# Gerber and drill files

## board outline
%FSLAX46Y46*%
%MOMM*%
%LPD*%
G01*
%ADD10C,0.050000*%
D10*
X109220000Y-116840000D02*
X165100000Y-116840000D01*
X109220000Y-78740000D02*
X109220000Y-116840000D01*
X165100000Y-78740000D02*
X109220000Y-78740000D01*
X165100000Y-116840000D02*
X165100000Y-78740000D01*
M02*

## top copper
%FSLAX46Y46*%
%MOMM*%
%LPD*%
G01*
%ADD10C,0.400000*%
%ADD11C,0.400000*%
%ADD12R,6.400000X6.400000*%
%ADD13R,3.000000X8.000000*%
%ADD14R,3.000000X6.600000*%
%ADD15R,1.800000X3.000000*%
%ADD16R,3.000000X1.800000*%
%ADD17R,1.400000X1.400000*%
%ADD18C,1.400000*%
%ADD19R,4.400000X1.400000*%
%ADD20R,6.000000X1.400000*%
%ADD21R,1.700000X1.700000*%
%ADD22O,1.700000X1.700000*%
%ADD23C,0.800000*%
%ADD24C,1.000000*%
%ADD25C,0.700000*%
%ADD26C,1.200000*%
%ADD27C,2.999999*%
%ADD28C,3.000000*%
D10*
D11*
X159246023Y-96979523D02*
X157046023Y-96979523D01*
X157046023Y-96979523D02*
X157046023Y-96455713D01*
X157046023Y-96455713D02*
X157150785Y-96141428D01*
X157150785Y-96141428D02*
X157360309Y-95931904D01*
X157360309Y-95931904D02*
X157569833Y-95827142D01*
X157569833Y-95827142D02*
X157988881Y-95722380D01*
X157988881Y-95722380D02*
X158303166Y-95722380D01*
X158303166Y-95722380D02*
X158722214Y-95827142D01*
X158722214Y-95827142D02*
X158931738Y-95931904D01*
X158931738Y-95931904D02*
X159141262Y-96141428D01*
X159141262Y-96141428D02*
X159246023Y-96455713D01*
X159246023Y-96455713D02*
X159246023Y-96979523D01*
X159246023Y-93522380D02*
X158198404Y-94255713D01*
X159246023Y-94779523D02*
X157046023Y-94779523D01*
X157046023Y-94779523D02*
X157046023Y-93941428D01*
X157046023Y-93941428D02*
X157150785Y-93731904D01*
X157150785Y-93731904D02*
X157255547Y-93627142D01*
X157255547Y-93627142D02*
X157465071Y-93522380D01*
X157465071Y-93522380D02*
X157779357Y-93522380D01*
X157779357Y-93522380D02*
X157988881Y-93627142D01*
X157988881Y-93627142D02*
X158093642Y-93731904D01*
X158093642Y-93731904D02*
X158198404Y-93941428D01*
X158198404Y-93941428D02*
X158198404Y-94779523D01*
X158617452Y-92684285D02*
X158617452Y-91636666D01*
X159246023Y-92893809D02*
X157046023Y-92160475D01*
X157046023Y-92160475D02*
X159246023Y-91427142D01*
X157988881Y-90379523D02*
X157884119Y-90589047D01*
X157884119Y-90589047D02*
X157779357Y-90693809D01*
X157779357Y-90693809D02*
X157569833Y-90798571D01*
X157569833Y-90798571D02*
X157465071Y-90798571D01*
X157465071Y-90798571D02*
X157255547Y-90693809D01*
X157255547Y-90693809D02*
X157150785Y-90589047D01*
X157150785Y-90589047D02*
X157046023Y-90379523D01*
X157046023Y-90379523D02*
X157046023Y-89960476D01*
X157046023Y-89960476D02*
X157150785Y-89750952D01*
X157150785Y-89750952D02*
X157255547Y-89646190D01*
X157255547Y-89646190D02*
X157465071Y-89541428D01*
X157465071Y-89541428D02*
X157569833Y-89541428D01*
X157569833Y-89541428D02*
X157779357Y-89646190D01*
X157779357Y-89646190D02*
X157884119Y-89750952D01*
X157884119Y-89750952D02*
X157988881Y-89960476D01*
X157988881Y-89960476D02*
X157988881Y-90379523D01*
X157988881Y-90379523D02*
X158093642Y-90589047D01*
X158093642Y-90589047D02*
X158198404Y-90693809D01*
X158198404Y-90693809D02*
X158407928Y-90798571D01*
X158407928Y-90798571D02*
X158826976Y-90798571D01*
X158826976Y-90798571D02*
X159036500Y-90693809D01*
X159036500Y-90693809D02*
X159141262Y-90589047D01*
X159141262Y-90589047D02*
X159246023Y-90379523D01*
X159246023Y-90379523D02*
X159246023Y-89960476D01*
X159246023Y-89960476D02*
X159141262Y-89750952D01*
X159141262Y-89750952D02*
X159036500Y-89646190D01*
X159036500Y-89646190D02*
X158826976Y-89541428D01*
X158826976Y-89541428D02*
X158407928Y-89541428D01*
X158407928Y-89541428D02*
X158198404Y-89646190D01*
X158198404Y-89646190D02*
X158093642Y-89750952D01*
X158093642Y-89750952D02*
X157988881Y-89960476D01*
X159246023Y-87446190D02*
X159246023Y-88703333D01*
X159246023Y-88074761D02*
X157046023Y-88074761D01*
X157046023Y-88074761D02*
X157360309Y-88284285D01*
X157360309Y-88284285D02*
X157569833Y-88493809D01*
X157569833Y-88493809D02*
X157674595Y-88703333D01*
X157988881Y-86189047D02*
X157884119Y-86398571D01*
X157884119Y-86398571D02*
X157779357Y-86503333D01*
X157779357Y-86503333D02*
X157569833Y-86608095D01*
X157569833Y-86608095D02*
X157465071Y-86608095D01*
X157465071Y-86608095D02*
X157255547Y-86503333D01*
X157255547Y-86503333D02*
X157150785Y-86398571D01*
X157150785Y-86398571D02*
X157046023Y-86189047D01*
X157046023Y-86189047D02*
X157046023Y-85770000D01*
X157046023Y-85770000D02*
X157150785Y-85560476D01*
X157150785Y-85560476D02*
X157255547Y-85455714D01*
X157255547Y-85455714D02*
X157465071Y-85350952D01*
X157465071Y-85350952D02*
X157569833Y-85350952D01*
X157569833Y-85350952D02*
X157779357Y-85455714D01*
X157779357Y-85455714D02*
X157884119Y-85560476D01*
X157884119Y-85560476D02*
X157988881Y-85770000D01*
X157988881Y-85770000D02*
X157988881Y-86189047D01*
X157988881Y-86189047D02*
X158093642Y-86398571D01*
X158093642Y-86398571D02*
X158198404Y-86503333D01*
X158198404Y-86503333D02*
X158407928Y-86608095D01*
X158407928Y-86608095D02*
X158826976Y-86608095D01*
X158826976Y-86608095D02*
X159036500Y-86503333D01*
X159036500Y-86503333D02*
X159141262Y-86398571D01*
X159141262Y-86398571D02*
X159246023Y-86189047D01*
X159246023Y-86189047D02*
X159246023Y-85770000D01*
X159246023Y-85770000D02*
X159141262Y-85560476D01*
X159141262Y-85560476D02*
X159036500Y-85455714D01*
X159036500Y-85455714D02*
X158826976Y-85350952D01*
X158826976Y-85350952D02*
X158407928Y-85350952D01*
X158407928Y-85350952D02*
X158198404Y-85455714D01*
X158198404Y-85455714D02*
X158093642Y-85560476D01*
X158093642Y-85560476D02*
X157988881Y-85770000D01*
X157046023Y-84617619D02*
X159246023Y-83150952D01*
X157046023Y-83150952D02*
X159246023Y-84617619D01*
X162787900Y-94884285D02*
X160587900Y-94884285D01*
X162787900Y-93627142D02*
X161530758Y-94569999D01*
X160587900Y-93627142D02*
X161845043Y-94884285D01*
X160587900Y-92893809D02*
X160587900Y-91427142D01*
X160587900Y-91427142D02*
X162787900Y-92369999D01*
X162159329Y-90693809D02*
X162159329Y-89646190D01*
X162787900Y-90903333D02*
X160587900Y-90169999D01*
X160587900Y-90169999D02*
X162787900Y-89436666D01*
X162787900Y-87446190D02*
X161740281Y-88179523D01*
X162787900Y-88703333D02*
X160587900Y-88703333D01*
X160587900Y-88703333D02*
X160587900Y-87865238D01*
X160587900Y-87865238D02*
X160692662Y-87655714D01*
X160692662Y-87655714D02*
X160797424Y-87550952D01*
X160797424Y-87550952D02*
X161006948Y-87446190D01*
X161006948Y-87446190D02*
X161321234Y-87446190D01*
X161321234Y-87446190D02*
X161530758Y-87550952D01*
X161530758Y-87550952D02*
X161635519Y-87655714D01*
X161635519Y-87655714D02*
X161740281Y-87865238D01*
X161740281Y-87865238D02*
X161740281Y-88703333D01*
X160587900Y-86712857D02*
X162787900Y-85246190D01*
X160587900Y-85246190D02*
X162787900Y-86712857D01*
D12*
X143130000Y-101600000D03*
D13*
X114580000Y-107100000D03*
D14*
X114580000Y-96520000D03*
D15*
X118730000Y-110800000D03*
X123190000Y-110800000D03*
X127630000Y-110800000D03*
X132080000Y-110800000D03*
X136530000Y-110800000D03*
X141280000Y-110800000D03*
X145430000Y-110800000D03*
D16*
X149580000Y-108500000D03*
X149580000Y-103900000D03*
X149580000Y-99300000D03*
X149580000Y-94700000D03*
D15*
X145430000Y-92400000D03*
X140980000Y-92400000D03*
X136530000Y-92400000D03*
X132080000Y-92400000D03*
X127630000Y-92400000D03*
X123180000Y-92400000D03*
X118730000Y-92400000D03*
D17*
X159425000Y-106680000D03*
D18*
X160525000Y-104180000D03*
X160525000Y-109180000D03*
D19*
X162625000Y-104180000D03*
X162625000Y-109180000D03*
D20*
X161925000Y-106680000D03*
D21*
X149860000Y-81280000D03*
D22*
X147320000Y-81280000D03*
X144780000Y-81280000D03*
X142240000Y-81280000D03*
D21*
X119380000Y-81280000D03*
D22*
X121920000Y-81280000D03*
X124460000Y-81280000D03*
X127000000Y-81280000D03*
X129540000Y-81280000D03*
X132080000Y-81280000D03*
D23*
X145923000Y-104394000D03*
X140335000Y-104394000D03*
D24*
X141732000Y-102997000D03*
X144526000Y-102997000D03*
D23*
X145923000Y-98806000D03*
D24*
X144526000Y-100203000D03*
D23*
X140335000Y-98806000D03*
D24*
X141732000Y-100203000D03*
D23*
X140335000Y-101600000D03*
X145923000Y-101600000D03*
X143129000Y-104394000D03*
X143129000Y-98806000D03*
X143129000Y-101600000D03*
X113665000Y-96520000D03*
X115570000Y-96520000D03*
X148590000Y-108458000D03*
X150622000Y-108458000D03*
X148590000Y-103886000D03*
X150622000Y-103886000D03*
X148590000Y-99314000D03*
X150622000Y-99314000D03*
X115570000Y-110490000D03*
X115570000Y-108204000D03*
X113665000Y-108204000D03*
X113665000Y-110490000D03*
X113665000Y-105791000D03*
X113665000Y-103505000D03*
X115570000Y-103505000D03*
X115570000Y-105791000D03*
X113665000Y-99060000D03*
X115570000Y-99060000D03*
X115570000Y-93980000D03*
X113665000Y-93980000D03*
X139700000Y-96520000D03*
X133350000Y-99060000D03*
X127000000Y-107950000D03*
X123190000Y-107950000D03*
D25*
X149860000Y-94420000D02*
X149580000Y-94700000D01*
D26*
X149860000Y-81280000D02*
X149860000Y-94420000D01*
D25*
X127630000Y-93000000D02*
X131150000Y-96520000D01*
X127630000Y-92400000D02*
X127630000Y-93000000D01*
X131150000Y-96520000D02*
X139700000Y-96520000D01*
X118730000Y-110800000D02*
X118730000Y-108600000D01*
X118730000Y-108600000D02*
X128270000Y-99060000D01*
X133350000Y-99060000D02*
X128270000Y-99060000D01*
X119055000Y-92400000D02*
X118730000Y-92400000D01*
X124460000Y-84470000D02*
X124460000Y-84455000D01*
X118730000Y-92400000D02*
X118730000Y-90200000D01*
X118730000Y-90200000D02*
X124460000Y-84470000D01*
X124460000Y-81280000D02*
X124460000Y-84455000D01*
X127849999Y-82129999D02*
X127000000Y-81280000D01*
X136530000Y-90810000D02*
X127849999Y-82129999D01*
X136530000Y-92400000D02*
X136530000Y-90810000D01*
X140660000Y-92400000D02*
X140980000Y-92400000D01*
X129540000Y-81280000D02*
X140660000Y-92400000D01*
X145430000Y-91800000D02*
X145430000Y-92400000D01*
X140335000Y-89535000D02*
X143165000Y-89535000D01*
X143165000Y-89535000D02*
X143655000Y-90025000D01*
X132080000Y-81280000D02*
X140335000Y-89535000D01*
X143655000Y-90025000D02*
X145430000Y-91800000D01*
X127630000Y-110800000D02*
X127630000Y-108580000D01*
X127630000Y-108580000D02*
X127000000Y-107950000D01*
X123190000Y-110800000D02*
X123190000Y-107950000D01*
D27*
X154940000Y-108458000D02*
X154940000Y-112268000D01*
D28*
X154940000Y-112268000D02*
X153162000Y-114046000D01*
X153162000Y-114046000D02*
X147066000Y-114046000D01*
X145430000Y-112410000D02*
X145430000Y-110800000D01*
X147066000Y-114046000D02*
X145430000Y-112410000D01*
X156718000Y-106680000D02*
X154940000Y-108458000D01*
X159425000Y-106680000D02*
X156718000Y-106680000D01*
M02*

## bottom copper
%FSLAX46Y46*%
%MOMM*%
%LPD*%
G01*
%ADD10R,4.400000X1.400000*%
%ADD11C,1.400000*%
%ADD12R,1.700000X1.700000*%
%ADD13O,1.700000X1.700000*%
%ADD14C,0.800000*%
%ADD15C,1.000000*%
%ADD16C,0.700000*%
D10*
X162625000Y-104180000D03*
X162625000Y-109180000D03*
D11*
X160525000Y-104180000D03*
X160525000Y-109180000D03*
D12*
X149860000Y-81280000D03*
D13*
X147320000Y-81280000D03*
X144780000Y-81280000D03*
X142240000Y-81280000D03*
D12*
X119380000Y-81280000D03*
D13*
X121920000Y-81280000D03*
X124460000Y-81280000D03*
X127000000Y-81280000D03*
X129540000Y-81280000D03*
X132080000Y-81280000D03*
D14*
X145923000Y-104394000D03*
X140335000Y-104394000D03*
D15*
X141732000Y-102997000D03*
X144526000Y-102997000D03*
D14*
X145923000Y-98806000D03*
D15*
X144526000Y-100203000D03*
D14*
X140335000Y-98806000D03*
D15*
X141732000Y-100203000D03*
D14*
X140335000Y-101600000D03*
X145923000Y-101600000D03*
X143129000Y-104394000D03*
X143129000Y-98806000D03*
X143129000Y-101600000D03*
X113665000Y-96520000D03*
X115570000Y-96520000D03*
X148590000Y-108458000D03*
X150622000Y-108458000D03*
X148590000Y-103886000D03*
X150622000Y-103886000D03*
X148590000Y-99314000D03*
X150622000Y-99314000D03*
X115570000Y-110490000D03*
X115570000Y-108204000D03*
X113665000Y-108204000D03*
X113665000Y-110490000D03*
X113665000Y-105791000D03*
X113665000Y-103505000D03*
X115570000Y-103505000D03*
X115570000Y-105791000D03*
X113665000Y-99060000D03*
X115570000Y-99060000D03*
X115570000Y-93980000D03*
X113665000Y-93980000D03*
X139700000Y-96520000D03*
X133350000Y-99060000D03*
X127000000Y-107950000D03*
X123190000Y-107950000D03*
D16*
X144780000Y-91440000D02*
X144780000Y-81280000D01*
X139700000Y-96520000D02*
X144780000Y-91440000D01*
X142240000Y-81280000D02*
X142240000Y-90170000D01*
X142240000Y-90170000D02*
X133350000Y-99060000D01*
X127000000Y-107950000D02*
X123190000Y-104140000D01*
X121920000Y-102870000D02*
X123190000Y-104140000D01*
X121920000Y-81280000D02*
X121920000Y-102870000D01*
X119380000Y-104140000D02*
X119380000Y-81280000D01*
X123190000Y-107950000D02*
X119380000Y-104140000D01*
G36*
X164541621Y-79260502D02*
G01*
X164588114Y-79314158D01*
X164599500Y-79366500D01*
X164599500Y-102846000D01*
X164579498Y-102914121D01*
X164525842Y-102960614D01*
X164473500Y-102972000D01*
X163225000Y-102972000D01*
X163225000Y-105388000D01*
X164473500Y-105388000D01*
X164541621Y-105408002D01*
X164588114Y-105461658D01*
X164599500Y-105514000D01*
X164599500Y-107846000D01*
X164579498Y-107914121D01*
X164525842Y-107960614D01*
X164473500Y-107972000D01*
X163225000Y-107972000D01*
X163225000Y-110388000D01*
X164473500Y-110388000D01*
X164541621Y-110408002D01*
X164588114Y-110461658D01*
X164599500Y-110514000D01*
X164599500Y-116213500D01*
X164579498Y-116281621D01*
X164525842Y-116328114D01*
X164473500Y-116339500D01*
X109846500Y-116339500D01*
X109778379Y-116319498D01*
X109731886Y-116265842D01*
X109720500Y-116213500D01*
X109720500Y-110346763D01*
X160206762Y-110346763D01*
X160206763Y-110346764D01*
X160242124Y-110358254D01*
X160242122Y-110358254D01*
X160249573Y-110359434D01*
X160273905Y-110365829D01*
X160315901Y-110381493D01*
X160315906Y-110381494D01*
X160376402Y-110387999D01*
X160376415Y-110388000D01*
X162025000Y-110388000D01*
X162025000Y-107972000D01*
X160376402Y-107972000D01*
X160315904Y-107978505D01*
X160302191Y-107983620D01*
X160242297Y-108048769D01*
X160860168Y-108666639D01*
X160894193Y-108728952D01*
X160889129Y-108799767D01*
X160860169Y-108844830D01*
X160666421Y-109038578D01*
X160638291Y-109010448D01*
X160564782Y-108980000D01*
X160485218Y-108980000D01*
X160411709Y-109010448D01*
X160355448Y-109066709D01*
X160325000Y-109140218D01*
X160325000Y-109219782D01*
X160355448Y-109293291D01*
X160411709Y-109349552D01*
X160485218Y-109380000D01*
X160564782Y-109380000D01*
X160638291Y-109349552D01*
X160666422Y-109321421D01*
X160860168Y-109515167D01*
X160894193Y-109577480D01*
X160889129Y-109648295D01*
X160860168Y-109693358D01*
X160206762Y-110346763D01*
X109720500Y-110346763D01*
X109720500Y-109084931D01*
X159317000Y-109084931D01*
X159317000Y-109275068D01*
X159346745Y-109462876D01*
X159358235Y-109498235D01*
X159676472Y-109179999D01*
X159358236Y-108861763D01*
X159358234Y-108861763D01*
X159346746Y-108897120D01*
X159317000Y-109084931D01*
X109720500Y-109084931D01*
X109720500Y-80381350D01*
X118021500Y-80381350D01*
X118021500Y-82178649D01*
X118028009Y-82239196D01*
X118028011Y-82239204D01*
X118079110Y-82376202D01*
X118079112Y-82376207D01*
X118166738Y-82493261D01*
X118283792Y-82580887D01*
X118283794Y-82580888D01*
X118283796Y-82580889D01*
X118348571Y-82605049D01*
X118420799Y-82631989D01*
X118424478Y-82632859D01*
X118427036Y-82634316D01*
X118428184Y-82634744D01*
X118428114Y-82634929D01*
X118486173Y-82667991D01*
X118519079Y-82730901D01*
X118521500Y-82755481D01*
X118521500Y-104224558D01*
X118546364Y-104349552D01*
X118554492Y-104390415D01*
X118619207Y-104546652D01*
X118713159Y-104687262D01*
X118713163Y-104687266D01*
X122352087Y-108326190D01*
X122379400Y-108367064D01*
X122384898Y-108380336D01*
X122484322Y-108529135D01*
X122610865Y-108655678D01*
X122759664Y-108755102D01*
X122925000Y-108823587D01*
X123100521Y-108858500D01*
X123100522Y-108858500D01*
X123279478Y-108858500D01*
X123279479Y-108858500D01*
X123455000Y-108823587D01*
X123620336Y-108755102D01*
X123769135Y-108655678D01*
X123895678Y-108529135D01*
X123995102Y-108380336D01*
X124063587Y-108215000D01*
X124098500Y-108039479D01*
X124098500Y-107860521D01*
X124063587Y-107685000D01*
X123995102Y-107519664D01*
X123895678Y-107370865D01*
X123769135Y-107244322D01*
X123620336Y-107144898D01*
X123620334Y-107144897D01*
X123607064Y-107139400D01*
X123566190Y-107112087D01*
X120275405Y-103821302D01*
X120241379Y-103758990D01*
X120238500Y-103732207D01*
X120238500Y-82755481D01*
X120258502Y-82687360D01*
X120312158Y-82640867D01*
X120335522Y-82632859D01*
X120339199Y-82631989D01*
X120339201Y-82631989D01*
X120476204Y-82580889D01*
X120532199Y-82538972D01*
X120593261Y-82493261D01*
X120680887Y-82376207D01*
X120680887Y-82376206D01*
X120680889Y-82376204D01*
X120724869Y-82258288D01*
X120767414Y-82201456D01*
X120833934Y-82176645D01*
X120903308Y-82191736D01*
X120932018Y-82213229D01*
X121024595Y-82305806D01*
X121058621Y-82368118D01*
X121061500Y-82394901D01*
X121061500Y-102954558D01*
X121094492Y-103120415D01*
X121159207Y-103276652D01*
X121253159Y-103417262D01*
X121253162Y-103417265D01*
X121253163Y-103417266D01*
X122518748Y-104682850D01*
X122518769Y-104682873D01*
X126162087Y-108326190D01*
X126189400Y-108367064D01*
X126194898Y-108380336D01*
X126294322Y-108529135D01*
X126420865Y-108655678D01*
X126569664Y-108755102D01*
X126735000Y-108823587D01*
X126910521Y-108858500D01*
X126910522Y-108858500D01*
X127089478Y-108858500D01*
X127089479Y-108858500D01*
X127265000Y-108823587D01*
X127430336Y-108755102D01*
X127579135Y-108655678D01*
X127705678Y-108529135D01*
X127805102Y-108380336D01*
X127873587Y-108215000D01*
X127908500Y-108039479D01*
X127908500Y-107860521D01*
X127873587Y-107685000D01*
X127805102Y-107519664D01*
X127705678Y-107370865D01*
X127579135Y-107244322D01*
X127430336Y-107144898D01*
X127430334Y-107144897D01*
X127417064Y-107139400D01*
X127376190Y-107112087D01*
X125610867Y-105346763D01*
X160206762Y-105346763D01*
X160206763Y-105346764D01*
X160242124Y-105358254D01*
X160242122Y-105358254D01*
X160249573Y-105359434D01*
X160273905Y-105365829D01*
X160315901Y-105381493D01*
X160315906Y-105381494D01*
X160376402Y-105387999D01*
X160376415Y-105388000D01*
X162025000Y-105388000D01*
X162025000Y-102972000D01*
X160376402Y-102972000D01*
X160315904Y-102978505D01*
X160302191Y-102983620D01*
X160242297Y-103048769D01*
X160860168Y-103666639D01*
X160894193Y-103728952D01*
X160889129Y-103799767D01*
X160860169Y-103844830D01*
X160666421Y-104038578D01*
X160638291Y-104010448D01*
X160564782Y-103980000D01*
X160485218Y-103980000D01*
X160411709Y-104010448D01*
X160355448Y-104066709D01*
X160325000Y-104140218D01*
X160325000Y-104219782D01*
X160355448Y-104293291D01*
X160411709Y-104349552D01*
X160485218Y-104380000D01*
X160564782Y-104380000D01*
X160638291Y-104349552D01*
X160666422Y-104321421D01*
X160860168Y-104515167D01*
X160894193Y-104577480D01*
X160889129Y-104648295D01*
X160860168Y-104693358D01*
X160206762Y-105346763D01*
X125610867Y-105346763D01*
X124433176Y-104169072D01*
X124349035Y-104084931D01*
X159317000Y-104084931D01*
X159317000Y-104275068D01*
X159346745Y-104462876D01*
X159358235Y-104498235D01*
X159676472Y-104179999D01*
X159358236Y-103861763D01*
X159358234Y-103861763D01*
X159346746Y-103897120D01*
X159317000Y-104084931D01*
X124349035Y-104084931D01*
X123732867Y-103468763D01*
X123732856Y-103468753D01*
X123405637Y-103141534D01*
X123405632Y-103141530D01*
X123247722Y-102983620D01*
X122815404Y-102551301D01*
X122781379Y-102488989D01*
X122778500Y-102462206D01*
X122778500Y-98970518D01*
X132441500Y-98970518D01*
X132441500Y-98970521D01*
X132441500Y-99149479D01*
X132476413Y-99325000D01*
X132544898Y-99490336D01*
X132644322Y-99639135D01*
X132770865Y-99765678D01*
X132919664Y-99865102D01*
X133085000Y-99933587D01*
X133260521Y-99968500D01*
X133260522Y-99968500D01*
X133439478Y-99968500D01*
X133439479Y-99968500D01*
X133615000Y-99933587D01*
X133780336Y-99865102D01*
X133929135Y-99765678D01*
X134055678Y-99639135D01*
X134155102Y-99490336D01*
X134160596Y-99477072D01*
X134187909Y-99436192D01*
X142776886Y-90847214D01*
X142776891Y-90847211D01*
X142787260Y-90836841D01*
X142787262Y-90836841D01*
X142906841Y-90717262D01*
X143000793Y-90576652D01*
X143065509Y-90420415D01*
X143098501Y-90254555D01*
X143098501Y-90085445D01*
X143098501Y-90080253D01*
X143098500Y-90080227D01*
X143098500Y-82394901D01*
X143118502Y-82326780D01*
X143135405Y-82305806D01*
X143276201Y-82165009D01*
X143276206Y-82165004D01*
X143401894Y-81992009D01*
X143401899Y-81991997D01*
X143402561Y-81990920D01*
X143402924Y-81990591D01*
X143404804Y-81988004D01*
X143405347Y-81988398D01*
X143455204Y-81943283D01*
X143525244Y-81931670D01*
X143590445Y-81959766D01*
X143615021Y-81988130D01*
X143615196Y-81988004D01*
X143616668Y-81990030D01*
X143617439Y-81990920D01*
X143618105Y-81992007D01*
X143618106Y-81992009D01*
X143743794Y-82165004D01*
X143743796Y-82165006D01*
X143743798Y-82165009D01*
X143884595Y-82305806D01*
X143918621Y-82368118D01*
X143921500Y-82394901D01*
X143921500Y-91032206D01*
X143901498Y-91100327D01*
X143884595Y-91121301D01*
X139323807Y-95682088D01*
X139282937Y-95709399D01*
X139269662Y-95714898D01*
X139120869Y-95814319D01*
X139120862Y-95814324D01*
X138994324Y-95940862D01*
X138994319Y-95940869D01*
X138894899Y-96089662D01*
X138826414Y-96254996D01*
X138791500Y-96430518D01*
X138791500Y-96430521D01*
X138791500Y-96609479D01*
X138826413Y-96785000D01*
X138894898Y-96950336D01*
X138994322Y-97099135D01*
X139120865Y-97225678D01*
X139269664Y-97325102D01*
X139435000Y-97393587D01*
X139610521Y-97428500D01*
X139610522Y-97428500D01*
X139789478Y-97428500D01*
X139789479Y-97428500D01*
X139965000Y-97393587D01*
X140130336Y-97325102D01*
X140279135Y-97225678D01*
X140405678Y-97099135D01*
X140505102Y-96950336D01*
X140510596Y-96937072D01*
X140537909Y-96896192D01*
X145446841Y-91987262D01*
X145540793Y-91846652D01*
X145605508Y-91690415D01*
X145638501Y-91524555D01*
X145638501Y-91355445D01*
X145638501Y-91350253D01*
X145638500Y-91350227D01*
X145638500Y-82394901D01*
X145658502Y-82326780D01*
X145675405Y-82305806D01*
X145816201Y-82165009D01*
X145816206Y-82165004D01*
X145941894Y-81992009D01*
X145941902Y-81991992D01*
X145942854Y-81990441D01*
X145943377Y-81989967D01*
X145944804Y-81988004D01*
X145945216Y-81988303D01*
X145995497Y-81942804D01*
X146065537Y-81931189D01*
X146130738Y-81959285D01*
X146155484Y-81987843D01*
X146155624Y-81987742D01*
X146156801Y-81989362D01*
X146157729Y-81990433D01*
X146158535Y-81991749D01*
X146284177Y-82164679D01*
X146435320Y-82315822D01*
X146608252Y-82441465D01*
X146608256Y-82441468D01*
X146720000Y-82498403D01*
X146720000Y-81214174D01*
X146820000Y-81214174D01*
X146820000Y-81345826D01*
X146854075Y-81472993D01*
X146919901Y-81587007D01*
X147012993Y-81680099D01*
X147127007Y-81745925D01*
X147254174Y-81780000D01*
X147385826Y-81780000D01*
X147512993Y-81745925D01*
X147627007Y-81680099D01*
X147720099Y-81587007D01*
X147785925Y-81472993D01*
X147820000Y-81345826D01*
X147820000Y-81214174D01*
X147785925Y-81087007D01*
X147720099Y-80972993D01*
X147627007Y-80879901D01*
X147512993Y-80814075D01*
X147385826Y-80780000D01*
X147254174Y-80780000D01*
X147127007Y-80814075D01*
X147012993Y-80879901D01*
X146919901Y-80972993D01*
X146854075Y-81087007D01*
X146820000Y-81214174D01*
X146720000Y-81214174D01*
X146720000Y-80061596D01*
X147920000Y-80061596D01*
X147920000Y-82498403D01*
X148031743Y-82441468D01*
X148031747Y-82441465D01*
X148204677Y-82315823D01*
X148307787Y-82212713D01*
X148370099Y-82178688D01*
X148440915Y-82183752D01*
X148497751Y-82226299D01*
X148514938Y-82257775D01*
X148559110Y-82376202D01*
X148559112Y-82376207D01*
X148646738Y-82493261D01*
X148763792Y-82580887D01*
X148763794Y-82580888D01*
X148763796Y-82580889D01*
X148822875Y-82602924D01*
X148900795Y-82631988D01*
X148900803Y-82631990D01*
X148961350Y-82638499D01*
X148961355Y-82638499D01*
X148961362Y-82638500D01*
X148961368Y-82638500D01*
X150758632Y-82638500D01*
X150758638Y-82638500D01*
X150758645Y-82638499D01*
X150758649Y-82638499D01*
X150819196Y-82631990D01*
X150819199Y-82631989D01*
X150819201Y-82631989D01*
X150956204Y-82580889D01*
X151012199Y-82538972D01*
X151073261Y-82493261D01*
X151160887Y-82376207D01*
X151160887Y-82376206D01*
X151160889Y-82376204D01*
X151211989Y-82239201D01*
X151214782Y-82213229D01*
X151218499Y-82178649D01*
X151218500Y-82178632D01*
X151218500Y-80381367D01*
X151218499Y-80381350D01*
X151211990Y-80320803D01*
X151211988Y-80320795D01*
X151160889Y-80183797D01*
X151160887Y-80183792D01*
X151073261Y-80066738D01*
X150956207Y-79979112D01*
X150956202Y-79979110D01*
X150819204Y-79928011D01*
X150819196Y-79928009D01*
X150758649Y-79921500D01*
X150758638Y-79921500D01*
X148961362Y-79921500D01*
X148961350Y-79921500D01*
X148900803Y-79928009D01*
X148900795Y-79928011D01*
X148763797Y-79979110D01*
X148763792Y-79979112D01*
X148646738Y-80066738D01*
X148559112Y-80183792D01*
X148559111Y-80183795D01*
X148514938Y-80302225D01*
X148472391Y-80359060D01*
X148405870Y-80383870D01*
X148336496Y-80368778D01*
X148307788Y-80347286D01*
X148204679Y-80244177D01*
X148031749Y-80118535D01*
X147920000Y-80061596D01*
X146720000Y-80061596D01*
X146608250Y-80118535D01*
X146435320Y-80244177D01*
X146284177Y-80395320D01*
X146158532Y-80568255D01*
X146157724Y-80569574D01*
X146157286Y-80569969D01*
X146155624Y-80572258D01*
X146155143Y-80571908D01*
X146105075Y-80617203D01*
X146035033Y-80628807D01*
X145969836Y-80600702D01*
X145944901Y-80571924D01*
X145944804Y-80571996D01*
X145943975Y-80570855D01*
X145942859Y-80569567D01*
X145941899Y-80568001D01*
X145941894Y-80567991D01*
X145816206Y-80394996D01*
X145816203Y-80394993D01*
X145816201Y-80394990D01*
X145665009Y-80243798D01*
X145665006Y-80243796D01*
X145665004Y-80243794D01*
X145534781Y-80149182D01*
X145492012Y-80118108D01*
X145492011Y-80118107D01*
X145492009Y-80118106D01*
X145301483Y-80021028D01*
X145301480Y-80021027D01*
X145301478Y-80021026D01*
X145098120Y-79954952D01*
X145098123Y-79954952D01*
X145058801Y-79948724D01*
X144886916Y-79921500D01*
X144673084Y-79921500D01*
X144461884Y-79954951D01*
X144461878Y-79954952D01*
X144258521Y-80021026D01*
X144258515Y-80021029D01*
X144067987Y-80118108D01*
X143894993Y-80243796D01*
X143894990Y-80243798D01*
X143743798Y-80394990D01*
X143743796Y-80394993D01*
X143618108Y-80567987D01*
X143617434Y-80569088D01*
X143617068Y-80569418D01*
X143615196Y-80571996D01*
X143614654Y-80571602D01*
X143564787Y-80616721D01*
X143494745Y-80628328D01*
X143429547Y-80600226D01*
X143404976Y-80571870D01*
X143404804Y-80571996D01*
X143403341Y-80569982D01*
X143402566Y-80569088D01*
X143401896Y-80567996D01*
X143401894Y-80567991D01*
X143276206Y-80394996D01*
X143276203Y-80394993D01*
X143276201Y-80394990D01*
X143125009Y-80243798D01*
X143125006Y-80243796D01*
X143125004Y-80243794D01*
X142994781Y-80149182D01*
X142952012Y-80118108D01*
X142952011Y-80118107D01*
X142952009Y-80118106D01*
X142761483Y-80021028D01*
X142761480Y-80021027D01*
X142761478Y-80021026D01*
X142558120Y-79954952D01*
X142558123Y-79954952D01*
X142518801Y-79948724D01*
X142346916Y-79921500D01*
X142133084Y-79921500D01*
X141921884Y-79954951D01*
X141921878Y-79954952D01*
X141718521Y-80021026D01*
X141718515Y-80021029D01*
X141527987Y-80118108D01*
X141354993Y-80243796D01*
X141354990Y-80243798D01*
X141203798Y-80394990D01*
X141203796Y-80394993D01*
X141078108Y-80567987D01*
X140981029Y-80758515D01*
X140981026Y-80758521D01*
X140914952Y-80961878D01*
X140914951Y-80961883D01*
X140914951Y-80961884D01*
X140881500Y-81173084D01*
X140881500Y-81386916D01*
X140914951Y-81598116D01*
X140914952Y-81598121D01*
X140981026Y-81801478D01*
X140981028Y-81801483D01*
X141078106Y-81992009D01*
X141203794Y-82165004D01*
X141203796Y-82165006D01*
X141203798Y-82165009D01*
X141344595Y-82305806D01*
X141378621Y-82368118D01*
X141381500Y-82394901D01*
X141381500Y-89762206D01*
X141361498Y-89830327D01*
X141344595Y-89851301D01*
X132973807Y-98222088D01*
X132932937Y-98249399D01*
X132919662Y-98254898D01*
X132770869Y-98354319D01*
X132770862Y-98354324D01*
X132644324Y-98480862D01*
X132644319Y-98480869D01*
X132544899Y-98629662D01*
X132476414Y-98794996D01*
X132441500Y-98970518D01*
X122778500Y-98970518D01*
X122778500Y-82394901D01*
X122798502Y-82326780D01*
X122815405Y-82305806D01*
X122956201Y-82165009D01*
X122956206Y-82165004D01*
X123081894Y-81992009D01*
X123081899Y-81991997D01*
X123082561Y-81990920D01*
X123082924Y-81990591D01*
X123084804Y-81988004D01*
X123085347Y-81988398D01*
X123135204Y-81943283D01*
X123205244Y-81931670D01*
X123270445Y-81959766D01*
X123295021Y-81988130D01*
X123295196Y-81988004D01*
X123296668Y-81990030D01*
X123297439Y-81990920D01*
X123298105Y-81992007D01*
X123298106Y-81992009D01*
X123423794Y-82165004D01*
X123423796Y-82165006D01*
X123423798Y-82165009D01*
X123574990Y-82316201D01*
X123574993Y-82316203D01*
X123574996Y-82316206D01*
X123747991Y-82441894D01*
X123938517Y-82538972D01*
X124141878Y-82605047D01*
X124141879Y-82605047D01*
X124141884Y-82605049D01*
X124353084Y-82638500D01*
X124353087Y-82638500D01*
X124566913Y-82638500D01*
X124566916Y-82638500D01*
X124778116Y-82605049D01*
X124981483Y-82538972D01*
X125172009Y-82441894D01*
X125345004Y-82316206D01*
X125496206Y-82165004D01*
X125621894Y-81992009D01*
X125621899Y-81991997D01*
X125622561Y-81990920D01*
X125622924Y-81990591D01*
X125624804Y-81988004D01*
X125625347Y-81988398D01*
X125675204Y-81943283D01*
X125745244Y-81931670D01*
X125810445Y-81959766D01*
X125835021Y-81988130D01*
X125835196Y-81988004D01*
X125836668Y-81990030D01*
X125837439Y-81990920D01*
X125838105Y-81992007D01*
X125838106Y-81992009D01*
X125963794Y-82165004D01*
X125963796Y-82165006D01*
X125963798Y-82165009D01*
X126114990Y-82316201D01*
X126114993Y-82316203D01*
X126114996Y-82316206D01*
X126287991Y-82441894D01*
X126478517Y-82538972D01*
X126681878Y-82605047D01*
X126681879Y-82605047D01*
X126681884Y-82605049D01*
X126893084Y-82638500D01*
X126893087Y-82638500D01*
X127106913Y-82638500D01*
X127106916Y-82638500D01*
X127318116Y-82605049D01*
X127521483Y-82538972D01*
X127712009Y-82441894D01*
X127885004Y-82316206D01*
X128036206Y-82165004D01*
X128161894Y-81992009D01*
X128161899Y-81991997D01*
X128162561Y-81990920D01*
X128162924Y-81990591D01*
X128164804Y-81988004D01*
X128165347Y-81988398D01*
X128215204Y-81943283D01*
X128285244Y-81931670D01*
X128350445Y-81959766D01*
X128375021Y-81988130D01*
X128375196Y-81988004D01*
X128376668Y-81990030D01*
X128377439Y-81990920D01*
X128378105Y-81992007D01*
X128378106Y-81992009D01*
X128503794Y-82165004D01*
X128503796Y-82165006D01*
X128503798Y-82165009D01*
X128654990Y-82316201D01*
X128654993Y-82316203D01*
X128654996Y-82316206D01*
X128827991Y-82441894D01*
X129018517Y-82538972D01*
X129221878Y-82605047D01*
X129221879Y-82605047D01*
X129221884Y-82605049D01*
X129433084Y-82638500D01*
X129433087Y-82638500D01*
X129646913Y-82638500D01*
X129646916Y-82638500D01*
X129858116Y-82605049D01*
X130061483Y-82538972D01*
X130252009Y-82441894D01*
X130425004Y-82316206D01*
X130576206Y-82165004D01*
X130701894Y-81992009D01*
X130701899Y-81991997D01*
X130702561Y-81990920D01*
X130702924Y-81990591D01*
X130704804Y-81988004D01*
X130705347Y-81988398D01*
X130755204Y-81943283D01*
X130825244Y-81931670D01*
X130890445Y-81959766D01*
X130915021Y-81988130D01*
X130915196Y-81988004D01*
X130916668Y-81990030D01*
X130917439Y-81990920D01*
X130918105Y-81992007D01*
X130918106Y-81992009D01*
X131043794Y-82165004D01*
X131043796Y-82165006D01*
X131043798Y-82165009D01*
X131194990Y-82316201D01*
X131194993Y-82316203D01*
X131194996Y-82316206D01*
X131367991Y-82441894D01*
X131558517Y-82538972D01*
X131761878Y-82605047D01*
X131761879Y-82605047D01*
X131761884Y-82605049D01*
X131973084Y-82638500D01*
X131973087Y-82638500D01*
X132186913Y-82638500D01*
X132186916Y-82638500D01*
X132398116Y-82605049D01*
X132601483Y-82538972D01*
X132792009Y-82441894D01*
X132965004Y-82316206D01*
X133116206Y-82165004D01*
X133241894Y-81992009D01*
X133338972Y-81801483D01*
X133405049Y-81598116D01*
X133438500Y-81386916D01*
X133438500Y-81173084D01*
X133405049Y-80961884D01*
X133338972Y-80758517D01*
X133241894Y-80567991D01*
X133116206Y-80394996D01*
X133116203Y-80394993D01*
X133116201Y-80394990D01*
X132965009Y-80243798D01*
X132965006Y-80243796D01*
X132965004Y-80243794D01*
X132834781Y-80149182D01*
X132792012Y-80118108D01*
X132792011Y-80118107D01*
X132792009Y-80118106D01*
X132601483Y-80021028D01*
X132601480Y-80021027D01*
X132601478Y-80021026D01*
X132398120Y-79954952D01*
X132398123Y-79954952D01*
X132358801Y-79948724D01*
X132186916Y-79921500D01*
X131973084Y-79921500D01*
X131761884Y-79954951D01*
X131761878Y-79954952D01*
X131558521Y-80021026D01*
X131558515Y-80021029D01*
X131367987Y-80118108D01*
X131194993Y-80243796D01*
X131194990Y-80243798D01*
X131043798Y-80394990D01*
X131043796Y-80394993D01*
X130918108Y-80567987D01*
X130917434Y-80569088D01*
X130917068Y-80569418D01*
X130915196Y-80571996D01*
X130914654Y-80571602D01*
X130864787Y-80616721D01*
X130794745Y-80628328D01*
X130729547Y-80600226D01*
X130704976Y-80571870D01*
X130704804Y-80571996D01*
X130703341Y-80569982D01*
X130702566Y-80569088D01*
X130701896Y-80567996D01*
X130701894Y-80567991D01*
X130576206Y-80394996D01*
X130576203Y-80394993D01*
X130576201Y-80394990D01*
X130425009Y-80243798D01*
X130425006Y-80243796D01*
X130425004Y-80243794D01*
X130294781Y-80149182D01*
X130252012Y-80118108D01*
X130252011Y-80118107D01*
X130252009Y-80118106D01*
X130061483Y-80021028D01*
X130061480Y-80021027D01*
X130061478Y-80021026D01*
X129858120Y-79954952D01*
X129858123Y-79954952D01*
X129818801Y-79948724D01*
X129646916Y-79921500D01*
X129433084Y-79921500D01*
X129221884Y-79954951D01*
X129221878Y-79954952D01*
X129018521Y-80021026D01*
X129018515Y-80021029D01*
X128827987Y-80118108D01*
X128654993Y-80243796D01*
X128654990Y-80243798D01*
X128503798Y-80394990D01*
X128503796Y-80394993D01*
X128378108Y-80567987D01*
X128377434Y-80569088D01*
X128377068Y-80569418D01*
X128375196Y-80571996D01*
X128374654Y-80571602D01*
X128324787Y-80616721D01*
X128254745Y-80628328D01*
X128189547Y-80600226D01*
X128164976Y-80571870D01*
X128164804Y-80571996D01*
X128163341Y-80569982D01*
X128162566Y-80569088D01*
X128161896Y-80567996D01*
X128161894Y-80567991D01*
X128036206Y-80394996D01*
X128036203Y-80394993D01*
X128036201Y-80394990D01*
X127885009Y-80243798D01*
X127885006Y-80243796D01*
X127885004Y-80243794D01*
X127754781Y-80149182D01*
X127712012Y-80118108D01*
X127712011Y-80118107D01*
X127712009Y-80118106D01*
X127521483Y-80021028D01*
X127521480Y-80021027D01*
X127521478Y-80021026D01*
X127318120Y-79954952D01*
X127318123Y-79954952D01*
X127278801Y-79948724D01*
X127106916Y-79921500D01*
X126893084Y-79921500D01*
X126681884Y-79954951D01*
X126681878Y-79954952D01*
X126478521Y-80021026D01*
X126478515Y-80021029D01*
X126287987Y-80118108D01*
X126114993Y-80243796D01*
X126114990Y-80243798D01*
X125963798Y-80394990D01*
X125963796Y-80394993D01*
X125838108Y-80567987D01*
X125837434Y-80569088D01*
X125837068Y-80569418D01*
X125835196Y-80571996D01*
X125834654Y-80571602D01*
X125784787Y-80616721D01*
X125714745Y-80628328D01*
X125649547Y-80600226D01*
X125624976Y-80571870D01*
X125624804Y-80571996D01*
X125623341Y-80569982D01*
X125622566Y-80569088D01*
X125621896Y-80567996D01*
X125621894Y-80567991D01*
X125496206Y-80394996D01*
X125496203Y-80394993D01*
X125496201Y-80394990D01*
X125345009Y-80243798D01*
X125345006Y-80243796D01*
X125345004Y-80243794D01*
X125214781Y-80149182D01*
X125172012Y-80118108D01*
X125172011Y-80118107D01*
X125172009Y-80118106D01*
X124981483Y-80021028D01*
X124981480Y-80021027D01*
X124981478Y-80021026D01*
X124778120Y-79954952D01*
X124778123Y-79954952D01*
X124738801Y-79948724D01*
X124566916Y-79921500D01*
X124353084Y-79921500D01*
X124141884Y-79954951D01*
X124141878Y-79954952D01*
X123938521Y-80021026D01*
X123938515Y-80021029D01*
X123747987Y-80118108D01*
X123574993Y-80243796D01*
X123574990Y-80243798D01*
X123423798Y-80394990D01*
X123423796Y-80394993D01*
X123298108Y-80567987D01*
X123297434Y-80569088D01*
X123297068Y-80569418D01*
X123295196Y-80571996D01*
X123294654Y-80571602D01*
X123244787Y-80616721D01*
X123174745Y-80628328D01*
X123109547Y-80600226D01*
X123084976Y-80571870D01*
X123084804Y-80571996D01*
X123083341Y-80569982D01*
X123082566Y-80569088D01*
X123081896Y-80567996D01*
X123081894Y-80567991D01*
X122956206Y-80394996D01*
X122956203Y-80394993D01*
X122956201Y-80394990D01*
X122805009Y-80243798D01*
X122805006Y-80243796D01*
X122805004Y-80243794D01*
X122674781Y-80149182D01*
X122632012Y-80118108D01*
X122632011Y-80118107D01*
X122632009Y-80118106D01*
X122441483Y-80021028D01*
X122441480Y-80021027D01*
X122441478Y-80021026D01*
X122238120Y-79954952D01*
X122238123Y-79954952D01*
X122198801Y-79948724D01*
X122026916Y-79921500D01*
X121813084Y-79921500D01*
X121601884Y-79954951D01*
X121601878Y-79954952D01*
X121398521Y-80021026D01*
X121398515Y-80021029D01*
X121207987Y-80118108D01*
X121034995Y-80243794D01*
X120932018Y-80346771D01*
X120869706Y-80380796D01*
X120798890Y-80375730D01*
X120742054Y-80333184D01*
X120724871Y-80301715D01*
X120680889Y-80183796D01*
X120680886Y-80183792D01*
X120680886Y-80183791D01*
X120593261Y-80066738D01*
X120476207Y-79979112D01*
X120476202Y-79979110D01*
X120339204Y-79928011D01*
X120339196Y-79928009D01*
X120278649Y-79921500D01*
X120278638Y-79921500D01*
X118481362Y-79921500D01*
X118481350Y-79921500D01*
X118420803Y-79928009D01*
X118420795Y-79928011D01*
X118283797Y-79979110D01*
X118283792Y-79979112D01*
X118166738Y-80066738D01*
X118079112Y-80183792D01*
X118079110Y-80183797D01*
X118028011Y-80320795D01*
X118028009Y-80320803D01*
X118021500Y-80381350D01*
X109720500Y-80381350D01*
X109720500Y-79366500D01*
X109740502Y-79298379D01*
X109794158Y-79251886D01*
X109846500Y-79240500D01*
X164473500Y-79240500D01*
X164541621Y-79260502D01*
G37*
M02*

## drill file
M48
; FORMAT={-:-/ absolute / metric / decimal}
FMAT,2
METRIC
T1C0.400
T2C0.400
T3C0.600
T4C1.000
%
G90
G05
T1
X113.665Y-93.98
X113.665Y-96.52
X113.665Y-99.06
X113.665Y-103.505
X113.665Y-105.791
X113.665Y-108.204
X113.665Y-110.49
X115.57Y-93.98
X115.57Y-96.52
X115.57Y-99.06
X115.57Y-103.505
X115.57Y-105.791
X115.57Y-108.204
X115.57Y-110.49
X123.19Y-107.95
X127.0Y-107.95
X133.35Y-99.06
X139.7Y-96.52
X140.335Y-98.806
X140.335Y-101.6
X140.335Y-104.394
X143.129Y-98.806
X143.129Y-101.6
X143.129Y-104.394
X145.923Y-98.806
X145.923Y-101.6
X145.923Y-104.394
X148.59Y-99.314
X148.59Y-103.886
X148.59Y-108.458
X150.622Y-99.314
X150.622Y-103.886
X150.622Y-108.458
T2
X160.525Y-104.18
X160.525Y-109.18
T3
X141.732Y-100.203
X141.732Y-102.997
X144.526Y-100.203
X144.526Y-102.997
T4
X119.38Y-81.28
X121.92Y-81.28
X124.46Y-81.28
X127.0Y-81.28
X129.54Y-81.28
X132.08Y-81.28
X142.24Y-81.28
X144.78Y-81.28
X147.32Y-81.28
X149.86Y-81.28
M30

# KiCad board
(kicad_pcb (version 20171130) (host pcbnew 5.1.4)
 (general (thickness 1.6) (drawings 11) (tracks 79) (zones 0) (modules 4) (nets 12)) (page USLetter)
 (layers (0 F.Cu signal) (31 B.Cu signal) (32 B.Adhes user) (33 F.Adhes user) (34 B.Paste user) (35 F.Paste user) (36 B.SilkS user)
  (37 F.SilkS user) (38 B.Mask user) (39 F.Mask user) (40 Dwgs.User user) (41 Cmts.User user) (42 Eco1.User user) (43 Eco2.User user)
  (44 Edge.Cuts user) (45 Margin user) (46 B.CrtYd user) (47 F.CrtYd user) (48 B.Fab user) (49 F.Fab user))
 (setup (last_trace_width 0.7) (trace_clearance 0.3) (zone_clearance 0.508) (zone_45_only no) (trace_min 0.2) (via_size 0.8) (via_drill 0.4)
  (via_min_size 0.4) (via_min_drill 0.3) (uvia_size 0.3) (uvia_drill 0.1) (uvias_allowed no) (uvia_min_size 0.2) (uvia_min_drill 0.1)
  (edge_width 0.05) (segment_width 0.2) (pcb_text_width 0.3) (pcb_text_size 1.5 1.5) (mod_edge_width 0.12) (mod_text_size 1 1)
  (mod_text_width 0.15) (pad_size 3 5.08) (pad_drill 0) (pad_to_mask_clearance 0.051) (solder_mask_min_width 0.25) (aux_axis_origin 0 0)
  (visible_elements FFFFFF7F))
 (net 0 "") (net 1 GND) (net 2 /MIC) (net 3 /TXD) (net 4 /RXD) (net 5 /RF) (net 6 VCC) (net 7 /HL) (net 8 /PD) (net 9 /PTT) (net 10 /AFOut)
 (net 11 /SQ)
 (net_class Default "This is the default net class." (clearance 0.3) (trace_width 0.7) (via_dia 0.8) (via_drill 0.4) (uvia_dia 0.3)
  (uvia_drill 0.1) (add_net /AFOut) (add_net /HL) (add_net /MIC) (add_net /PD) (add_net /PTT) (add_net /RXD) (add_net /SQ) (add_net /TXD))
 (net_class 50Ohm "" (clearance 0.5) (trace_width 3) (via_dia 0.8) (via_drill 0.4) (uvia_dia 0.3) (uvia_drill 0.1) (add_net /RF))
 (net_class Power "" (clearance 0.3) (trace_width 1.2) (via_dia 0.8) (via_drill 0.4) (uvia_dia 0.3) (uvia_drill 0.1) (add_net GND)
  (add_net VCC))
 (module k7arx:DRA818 (layer F.Cu) (at 132.08 101.6)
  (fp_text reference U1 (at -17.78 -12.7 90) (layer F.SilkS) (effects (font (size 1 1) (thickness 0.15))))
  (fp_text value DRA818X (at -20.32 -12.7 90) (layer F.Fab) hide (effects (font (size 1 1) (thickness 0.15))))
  (pad 0 smd rect (at 11.05 0) (size 6.4 6.4) (layers F.Cu F.Paste F.Mask) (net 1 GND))
  (pad 0 smd rect (at -17.5 5.5) (size 3 8) (layers F.Cu F.Paste F.Mask) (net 1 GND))
  (pad 0 smd rect (at -17.5 -5.08) (size 3 6.6) (layers F.Cu F.Paste F.Mask) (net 1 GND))
  (pad 18 smd rect (at -13.35 9.2) (size 1.8 3) (layers F.Cu F.Paste F.Mask) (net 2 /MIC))
  (pad 17 smd rect (at -8.89 9.2) (size 1.8 3) (layers F.Cu F.Paste F.Mask) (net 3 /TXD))
  (pad 16 smd rect (at -4.45 9.2) (size 1.8 3) (layers F.Cu F.Paste F.Mask) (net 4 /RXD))
  (pad 15 smd rect (at 0 9.2) (size 1.8 3) (layers F.Cu F.Paste F.Mask))
  (pad 14 smd rect (at 4.45 9.2) (size 1.8 3) (layers F.Cu F.Paste F.Mask))
  (pad 13 smd rect (at 9.2 9.2) (size 1.8 3) (layers F.Cu F.Paste F.Mask))
  (pad 12 smd rect (at 13.35 9.2) (size 1.8 3) (layers F.Cu F.Paste F.Mask) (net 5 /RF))
  (pad 11 smd rect (at 17.5 6.9) (size 3 1.8) (layers F.Cu F.Paste F.Mask) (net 1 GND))
  (pad 10 smd rect (at 17.5 2.3) (size 3 1.8) (layers F.Cu F.Paste F.Mask) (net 1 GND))
  (pad 9 smd rect (at 17.5 -2.3) (size 3 1.8) (layers F.Cu F.Paste F.Mask) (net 1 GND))
  (pad 8 smd rect (at 17.5 -6.9) (size 3 1.8) (layers F.Cu F.Paste F.Mask) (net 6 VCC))
  (pad 7 smd rect (at 13.35 -9.2) (size 1.8 3) (layers F.Cu F.Paste F.Mask) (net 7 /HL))
  (pad 6 smd rect (at 8.9 -9.2) (size 1.8 3) (layers F.Cu F.Paste F.Mask) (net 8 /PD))
  (pad 5 smd rect (at 4.45 -9.2) (size 1.8 3) (layers F.Cu F.Paste F.Mask) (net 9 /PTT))
  (pad 4 smd rect (at 0 -9.2) (size 1.8 3) (layers F.Cu F.Paste F.Mask))
  (pad 3 smd rect (at -4.45 -9.2) (size 1.8 3) (layers F.Cu F.Paste F.Mask) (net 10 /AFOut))
  (pad 2 smd rect (at -8.9 -9.2) (size 1.8 3) (layers F.Cu F.Paste F.Mask))
  (pad 1 smd rect (at -13.35 -9.2) (size 1.8 3) (layers F.Cu F.Paste F.Mask) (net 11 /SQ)))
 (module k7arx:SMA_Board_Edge (layer F.Cu) (at 164.925 106.68 180)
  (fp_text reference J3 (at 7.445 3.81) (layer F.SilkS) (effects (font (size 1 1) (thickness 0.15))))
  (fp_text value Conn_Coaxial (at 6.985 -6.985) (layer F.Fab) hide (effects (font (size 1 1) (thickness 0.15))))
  (pad 1 smd rect (at 5.5 0 180) (size 1.4 1.4) (layers F.Cu F.Paste F.Mask) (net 5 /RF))
  (pad 2 smd rect (at 2.3 2.5 180) (size 4.4 1.4) (layers B.Cu B.Paste B.Mask) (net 1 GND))
  (pad 2 smd rect (at 2.3 -2.5 180) (size 4.4 1.4) (layers B.Cu B.Paste B.Mask) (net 1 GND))
  (pad 2 thru_hole circle (at 4.4 2.5 180) (size 1.4 1.4) (drill 0.4) (layers *.Cu *.Mask) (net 1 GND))
  (pad 2 thru_hole circle (at 4.4 -2.5 180) (size 1.4 1.4) (drill 0.4) (layers *.Cu *.Mask) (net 1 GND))
  (pad 2 smd rect (at 2.3 2.5 180) (size 4.4 1.4) (layers F.Cu F.Paste F.Mask) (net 1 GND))
  (pad 2 smd rect (at 2.3 -2.5 180) (size 4.4 1.4) (layers F.Cu F.Paste F.Mask) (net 1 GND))
  (pad 1 smd rect (at 3 0 180) (size 6 1.4) (layers F.Cu F.Paste F.Mask) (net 5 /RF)))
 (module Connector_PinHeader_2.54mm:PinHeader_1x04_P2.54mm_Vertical (layer F.Cu) (at 149.86 81.28 270)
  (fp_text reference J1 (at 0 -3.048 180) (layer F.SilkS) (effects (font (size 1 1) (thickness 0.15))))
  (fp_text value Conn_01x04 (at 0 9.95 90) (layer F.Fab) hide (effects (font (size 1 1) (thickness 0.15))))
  (pad 1 thru_hole rect (at 0 0 270) (size 1.7 1.7) (drill 1) (layers *.Cu *.Mask) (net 6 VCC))
  (pad 2 thru_hole oval (at 0 2.54 270) (size 1.7 1.7) (drill 1) (layers *.Cu *.Mask) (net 1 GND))
  (pad 3 thru_hole oval (at 0 5.08 270) (size 1.7 1.7) (drill 1) (layers *.Cu *.Mask) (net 10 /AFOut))
  (pad 4 thru_hole oval (at 0 7.62 270) (size 1.7 1.7) (drill 1) (layers *.Cu *.Mask) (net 2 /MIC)))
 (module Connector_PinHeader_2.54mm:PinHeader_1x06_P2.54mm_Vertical (layer F.Cu) (at 119.38 81.28 90)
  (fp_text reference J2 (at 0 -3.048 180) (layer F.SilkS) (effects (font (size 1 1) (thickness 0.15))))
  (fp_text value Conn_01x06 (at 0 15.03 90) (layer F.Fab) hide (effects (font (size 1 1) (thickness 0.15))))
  (pad 1 thru_hole rect (at 0 0 90) (size 1.7 1.7) (drill 1) (layers *.Cu *.Mask) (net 3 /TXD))
  (pad 2 thru_hole oval (at 0 2.54 90) (size 1.7 1.7) (drill 1) (layers *.Cu *.Mask) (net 4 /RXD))
  (pad 3 thru_hole oval (at 0 5.08 90) (size 1.7 1.7) (drill 1) (layers *.Cu *.Mask) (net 11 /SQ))
  (pad 4 thru_hole oval (at 0 7.62 90) (size 1.7 1.7) (drill 1) (layers *.Cu *.Mask) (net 9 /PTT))
  (pad 5 thru_hole oval (at 0 10.16 90) (size 1.7 1.7) (drill 1) (layers *.Cu *.Mask) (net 8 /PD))
  (pad 6 thru_hole oval (at 0 12.7 90) (size 1.7 1.7) (drill 1) (layers *.Cu *.Mask) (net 7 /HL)))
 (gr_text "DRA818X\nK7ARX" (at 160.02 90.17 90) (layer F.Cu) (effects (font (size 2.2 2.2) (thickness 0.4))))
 (gr_line (start 109.22 116.84) (end 165.1 116.84) (layer Edge.Cuts) (width 0.05))
 (gr_line (start 109.22 78.74) (end 109.22 116.84) (layer Edge.Cuts) (width 0.05))
 (gr_line (start 165.1 78.74) (end 109.22 78.74) (layer Edge.Cuts) (width 0.05))
 (gr_line (start 165.1 116.84) (end 165.1 78.74) (layer Edge.Cuts) (width 0.05))
 (via (at 145.923 104.394) (size 0.8) (drill 0.4) (layers F.Cu B.Cu) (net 1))
 (via (at 140.335 104.394) (size 0.8) (drill 0.4) (layers F.Cu B.Cu) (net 1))
 (via (at 141.732 102.997) (size 1) (drill 0.6) (layers F.Cu B.Cu) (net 1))
 (via (at 144.526 102.997) (size 1) (drill 0.6) (layers F.Cu B.Cu) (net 1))
 (via (at 145.923 98.806) (size 0.8) (drill 0.4) (layers F.Cu B.Cu) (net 1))
 (via (at 144.526 100.203) (size 1) (drill 0.6) (layers F.Cu B.Cu) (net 1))
 (via (at 140.335 98.806) (size 0.8) (drill 0.4) (layers F.Cu B.Cu) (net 1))
 (via (at 141.732 100.203) (size 1) (drill 0.6) (layers F.Cu B.Cu) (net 1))
 (via (at 140.335 101.6) (size 0.8) (drill 0.4) (layers F.Cu B.Cu) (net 1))
 (via (at 145.923 101.6) (size 0.8) (drill 0.4) (layers F.Cu B.Cu) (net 1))
 (via (at 143.129 104.394) (size 0.8) (drill 0.4) (layers F.Cu B.Cu) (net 1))
 (via (at 143.129 98.806) (size 0.8) (drill 0.4) (layers F.Cu B.Cu) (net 1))
 (via (at 143.129 101.6) (size 0.8) (drill 0.4) (layers F.Cu B.Cu) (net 1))
 (via (at 113.665 96.52) (size 0.8) (drill 0.4) (layers F.Cu B.Cu) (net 1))
 (via (at 115.57 96.52) (size 0.8) (drill 0.4) (layers F.Cu B.Cu) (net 1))
 (via (at 148.59 108.458) (size 0.8) (drill 0.4) (layers F.Cu B.Cu) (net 1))
 (via (at 150.622 108.458) (size 0.8) (drill 0.4) (layers F.Cu B.Cu) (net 1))
 (via (at 148.59 103.886) (size 0.8) (drill 0.4) (layers F.Cu B.Cu) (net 1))
 (via (at 150.622 103.886) (size 0.8) (drill 0.4) (layers F.Cu B.Cu) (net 1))
 (via (at 148.59 99.314) (size 0.8) (drill 0.4) (layers F.Cu B.Cu) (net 1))
 (via (at 150.622 99.314) (size 0.8) (drill 0.4) (layers F.Cu B.Cu) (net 1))
 (via (at 115.57 110.49) (size 0.8) (drill 0.4) (layers F.Cu B.Cu) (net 1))
 (via (at 115.57 108.204) (size 0.8) (drill 0.4) (layers F.Cu B.Cu) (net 1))
 (via (at 113.665 108.204) (size 0.8) (drill 0.4) (layers F.Cu B.Cu) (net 1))
 (via (at 113.665 110.49) (size 0.8) (drill 0.4) (layers F.Cu B.Cu) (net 1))
 (via (at 113.665 105.791) (size 0.8) (drill 0.4) (layers F.Cu B.Cu) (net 1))
 (via (at 113.665 103.505) (size 0.8) (drill 0.4) (layers F.Cu B.Cu) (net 1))
 (via (at 115.57 103.505) (size 0.8) (drill 0.4) (layers F.Cu B.Cu) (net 1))
 (via (at 115.57 105.791) (size 0.8) (drill 0.4) (layers F.Cu B.Cu) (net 1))
 (via (at 113.665 99.06) (size 0.8) (drill 0.4) (layers F.Cu B.Cu) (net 1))
 (via (at 115.57 99.06) (size 0.8) (drill 0.4) (layers F.Cu B.Cu) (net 1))
 (via (at 115.57 93.98) (size 0.8) (drill 0.4) (layers F.Cu B.Cu) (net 1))
 (via (at 113.665 93.98) (size 0.8) (drill 0.4) (layers F.Cu B.Cu) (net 1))
 (segment (start 149.86 94.42) (end 149.58 94.7) (width 0.7) (layer F.Cu) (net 6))
 (segment (start 149.86 81.28) (end 149.86 94.42) (width 1.2) (layer F.Cu) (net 6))
 (segment (start 127.63 93) (end 131.15 96.52) (width 0.7) (layer F.Cu) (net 10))
 (segment (start 127.63 92.4) (end 127.63 93) (width 0.7) (layer F.Cu) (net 10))
 (via (at 139.7 96.52) (size 0.8) (drill 0.4) (layers F.Cu B.Cu) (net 10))
 (segment (start 144.78 91.44) (end 144.78 81.28) (width 0.7) (layer B.Cu) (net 10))
 (segment (start 139.7 96.52) (end 144.78 91.44) (width 0.7) (layer B.Cu) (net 10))
 (segment (start 131.15 96.52) (end 139.7 96.52) (width 0.7) (layer F.Cu) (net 10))
 (segment (start 118.73 110.8) (end 118.73 108.6) (width 0.7) (layer F.Cu) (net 2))
 (via (at 133.35 99.06) (size 0.8) (drill 0.4) (layers F.Cu B.Cu) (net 2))
 (segment (start 118.73 108.6) (end 128.27 99.06) (width 0.7) (layer F.Cu) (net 2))
 (segment (start 142.24 81.28) (end 142.24 90.17) (width 0.7) (layer B.Cu) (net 2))
 (segment (start 142.24 90.17) (end 133.35 99.06) (width 0.7) (layer B.Cu) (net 2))
 (segment (start 133.35 99.06) (end 128.27 99.06) (width 0.7) (layer F.Cu) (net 2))
 (segment (start 119.055 92.4) (end 118.73 92.4) (width 0.7) (layer F.Cu) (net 11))
 (segment (start 124.46 84.47) (end 124.46 84.455) (width 0.7) (layer F.Cu) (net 11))
 (segment (start 118.73 92.4) (end 118.73 90.2) (width 0.7) (layer F.Cu) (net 11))
 (segment (start 118.73 90.2) (end 124.46 84.47) (width 0.7) (layer F.Cu) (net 11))
 (segment (start 124.46 81.28) (end 124.46 84.455) (width 0.7) (layer F.Cu) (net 11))
 (segment (start 127.849999 82.129999) (end 127 81.28) (width 0.7) (layer F.Cu) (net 9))
 (segment (start 136.53 90.81) (end 127.849999 82.129999) (width 0.7) (layer F.Cu) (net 9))
 (segment (start 136.53 92.4) (end 136.53 90.81) (width 0.7) (layer F.Cu) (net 9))
 (segment (start 140.66 92.4) (end 140.98 92.4) (width 0.7) (layer F.Cu) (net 8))
 (segment (start 129.54 81.28) (end 140.66 92.4) (width 0.7) (layer F.Cu) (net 8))
 (segment (start 145.43 91.8) (end 145.43 92.4) (width 0.7) (layer F.Cu) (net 7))
 (segment (start 140.335 89.535) (end 143.165 89.535) (width 0.7) (layer F.Cu) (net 7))
 (segment (start 143.165 89.535) (end 143.655 90.025) (width 0.7) (layer F.Cu) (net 7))
 (segment (start 132.08 81.28) (end 140.335 89.535) (width 0.7) (layer F.Cu) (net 7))
 (segment (start 143.655 90.025) (end 145.43 91.8) (width 0.7) (layer F.Cu) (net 7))
 (segment (start 127.63 110.8) (end 127.63 108.58) (width 0.7) (layer F.Cu) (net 4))
 (via (at 127 107.95) (size 0.8) (drill 0.4) (layers F.Cu B.Cu) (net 4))
 (segment (start 127.63 108.58) (end 127 107.95) (width 0.7) (layer F.Cu) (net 4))
 (segment (start 127 107.95) (end 123.19 104.14) (width 0.7) (layer B.Cu) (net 4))
 (segment (start 121.92 102.87) (end 123.19 104.14) (width 0.7) (layer B.Cu) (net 4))
 (segment (start 121.92 81.28) (end 121.92 102.87) (width 0.7) (layer B.Cu) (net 4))
 (via (at 123.19 107.95) (size 0.8) (drill 0.4) (layers F.Cu B.Cu) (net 3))
 (segment (start 123.19 110.8) (end 123.19 107.95) (width 0.7) (layer F.Cu) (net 3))
 (segment (start 119.38 104.14) (end 119.38 81.28) (width 0.7) (layer B.Cu) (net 3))
 (segment (start 123.19 107.95) (end 119.38 104.14) (width 0.7) (layer B.Cu) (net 3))
 (segment (start 154.94 108.458) (end 154.94 112.268) (width 2.999999) (layer F.Cu) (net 5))
 (segment (start 154.94 112.268) (end 153.162 114.046) (width 3) (layer F.Cu) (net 5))
 (segment (start 153.162 114.046) (end 147.066 114.046) (width 3) (layer F.Cu) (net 5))
 (segment (start 145.43 112.41) (end 145.43 110.8) (width 3) (layer F.Cu) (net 5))
 (segment (start 147.066 114.046) (end 145.43 112.41) (width 3) (layer F.Cu) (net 5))
 (segment (start 156.718 106.68) (end 154.94 108.458) (width 3) (layer F.Cu) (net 5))
 (segment (start 159.425 106.68) (end 156.718 106.68) (width 3) (layer F.Cu) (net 5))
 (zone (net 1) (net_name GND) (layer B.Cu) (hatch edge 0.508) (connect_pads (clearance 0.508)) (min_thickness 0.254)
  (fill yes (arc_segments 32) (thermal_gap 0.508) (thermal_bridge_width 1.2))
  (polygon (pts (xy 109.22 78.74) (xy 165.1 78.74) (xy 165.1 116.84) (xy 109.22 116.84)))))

